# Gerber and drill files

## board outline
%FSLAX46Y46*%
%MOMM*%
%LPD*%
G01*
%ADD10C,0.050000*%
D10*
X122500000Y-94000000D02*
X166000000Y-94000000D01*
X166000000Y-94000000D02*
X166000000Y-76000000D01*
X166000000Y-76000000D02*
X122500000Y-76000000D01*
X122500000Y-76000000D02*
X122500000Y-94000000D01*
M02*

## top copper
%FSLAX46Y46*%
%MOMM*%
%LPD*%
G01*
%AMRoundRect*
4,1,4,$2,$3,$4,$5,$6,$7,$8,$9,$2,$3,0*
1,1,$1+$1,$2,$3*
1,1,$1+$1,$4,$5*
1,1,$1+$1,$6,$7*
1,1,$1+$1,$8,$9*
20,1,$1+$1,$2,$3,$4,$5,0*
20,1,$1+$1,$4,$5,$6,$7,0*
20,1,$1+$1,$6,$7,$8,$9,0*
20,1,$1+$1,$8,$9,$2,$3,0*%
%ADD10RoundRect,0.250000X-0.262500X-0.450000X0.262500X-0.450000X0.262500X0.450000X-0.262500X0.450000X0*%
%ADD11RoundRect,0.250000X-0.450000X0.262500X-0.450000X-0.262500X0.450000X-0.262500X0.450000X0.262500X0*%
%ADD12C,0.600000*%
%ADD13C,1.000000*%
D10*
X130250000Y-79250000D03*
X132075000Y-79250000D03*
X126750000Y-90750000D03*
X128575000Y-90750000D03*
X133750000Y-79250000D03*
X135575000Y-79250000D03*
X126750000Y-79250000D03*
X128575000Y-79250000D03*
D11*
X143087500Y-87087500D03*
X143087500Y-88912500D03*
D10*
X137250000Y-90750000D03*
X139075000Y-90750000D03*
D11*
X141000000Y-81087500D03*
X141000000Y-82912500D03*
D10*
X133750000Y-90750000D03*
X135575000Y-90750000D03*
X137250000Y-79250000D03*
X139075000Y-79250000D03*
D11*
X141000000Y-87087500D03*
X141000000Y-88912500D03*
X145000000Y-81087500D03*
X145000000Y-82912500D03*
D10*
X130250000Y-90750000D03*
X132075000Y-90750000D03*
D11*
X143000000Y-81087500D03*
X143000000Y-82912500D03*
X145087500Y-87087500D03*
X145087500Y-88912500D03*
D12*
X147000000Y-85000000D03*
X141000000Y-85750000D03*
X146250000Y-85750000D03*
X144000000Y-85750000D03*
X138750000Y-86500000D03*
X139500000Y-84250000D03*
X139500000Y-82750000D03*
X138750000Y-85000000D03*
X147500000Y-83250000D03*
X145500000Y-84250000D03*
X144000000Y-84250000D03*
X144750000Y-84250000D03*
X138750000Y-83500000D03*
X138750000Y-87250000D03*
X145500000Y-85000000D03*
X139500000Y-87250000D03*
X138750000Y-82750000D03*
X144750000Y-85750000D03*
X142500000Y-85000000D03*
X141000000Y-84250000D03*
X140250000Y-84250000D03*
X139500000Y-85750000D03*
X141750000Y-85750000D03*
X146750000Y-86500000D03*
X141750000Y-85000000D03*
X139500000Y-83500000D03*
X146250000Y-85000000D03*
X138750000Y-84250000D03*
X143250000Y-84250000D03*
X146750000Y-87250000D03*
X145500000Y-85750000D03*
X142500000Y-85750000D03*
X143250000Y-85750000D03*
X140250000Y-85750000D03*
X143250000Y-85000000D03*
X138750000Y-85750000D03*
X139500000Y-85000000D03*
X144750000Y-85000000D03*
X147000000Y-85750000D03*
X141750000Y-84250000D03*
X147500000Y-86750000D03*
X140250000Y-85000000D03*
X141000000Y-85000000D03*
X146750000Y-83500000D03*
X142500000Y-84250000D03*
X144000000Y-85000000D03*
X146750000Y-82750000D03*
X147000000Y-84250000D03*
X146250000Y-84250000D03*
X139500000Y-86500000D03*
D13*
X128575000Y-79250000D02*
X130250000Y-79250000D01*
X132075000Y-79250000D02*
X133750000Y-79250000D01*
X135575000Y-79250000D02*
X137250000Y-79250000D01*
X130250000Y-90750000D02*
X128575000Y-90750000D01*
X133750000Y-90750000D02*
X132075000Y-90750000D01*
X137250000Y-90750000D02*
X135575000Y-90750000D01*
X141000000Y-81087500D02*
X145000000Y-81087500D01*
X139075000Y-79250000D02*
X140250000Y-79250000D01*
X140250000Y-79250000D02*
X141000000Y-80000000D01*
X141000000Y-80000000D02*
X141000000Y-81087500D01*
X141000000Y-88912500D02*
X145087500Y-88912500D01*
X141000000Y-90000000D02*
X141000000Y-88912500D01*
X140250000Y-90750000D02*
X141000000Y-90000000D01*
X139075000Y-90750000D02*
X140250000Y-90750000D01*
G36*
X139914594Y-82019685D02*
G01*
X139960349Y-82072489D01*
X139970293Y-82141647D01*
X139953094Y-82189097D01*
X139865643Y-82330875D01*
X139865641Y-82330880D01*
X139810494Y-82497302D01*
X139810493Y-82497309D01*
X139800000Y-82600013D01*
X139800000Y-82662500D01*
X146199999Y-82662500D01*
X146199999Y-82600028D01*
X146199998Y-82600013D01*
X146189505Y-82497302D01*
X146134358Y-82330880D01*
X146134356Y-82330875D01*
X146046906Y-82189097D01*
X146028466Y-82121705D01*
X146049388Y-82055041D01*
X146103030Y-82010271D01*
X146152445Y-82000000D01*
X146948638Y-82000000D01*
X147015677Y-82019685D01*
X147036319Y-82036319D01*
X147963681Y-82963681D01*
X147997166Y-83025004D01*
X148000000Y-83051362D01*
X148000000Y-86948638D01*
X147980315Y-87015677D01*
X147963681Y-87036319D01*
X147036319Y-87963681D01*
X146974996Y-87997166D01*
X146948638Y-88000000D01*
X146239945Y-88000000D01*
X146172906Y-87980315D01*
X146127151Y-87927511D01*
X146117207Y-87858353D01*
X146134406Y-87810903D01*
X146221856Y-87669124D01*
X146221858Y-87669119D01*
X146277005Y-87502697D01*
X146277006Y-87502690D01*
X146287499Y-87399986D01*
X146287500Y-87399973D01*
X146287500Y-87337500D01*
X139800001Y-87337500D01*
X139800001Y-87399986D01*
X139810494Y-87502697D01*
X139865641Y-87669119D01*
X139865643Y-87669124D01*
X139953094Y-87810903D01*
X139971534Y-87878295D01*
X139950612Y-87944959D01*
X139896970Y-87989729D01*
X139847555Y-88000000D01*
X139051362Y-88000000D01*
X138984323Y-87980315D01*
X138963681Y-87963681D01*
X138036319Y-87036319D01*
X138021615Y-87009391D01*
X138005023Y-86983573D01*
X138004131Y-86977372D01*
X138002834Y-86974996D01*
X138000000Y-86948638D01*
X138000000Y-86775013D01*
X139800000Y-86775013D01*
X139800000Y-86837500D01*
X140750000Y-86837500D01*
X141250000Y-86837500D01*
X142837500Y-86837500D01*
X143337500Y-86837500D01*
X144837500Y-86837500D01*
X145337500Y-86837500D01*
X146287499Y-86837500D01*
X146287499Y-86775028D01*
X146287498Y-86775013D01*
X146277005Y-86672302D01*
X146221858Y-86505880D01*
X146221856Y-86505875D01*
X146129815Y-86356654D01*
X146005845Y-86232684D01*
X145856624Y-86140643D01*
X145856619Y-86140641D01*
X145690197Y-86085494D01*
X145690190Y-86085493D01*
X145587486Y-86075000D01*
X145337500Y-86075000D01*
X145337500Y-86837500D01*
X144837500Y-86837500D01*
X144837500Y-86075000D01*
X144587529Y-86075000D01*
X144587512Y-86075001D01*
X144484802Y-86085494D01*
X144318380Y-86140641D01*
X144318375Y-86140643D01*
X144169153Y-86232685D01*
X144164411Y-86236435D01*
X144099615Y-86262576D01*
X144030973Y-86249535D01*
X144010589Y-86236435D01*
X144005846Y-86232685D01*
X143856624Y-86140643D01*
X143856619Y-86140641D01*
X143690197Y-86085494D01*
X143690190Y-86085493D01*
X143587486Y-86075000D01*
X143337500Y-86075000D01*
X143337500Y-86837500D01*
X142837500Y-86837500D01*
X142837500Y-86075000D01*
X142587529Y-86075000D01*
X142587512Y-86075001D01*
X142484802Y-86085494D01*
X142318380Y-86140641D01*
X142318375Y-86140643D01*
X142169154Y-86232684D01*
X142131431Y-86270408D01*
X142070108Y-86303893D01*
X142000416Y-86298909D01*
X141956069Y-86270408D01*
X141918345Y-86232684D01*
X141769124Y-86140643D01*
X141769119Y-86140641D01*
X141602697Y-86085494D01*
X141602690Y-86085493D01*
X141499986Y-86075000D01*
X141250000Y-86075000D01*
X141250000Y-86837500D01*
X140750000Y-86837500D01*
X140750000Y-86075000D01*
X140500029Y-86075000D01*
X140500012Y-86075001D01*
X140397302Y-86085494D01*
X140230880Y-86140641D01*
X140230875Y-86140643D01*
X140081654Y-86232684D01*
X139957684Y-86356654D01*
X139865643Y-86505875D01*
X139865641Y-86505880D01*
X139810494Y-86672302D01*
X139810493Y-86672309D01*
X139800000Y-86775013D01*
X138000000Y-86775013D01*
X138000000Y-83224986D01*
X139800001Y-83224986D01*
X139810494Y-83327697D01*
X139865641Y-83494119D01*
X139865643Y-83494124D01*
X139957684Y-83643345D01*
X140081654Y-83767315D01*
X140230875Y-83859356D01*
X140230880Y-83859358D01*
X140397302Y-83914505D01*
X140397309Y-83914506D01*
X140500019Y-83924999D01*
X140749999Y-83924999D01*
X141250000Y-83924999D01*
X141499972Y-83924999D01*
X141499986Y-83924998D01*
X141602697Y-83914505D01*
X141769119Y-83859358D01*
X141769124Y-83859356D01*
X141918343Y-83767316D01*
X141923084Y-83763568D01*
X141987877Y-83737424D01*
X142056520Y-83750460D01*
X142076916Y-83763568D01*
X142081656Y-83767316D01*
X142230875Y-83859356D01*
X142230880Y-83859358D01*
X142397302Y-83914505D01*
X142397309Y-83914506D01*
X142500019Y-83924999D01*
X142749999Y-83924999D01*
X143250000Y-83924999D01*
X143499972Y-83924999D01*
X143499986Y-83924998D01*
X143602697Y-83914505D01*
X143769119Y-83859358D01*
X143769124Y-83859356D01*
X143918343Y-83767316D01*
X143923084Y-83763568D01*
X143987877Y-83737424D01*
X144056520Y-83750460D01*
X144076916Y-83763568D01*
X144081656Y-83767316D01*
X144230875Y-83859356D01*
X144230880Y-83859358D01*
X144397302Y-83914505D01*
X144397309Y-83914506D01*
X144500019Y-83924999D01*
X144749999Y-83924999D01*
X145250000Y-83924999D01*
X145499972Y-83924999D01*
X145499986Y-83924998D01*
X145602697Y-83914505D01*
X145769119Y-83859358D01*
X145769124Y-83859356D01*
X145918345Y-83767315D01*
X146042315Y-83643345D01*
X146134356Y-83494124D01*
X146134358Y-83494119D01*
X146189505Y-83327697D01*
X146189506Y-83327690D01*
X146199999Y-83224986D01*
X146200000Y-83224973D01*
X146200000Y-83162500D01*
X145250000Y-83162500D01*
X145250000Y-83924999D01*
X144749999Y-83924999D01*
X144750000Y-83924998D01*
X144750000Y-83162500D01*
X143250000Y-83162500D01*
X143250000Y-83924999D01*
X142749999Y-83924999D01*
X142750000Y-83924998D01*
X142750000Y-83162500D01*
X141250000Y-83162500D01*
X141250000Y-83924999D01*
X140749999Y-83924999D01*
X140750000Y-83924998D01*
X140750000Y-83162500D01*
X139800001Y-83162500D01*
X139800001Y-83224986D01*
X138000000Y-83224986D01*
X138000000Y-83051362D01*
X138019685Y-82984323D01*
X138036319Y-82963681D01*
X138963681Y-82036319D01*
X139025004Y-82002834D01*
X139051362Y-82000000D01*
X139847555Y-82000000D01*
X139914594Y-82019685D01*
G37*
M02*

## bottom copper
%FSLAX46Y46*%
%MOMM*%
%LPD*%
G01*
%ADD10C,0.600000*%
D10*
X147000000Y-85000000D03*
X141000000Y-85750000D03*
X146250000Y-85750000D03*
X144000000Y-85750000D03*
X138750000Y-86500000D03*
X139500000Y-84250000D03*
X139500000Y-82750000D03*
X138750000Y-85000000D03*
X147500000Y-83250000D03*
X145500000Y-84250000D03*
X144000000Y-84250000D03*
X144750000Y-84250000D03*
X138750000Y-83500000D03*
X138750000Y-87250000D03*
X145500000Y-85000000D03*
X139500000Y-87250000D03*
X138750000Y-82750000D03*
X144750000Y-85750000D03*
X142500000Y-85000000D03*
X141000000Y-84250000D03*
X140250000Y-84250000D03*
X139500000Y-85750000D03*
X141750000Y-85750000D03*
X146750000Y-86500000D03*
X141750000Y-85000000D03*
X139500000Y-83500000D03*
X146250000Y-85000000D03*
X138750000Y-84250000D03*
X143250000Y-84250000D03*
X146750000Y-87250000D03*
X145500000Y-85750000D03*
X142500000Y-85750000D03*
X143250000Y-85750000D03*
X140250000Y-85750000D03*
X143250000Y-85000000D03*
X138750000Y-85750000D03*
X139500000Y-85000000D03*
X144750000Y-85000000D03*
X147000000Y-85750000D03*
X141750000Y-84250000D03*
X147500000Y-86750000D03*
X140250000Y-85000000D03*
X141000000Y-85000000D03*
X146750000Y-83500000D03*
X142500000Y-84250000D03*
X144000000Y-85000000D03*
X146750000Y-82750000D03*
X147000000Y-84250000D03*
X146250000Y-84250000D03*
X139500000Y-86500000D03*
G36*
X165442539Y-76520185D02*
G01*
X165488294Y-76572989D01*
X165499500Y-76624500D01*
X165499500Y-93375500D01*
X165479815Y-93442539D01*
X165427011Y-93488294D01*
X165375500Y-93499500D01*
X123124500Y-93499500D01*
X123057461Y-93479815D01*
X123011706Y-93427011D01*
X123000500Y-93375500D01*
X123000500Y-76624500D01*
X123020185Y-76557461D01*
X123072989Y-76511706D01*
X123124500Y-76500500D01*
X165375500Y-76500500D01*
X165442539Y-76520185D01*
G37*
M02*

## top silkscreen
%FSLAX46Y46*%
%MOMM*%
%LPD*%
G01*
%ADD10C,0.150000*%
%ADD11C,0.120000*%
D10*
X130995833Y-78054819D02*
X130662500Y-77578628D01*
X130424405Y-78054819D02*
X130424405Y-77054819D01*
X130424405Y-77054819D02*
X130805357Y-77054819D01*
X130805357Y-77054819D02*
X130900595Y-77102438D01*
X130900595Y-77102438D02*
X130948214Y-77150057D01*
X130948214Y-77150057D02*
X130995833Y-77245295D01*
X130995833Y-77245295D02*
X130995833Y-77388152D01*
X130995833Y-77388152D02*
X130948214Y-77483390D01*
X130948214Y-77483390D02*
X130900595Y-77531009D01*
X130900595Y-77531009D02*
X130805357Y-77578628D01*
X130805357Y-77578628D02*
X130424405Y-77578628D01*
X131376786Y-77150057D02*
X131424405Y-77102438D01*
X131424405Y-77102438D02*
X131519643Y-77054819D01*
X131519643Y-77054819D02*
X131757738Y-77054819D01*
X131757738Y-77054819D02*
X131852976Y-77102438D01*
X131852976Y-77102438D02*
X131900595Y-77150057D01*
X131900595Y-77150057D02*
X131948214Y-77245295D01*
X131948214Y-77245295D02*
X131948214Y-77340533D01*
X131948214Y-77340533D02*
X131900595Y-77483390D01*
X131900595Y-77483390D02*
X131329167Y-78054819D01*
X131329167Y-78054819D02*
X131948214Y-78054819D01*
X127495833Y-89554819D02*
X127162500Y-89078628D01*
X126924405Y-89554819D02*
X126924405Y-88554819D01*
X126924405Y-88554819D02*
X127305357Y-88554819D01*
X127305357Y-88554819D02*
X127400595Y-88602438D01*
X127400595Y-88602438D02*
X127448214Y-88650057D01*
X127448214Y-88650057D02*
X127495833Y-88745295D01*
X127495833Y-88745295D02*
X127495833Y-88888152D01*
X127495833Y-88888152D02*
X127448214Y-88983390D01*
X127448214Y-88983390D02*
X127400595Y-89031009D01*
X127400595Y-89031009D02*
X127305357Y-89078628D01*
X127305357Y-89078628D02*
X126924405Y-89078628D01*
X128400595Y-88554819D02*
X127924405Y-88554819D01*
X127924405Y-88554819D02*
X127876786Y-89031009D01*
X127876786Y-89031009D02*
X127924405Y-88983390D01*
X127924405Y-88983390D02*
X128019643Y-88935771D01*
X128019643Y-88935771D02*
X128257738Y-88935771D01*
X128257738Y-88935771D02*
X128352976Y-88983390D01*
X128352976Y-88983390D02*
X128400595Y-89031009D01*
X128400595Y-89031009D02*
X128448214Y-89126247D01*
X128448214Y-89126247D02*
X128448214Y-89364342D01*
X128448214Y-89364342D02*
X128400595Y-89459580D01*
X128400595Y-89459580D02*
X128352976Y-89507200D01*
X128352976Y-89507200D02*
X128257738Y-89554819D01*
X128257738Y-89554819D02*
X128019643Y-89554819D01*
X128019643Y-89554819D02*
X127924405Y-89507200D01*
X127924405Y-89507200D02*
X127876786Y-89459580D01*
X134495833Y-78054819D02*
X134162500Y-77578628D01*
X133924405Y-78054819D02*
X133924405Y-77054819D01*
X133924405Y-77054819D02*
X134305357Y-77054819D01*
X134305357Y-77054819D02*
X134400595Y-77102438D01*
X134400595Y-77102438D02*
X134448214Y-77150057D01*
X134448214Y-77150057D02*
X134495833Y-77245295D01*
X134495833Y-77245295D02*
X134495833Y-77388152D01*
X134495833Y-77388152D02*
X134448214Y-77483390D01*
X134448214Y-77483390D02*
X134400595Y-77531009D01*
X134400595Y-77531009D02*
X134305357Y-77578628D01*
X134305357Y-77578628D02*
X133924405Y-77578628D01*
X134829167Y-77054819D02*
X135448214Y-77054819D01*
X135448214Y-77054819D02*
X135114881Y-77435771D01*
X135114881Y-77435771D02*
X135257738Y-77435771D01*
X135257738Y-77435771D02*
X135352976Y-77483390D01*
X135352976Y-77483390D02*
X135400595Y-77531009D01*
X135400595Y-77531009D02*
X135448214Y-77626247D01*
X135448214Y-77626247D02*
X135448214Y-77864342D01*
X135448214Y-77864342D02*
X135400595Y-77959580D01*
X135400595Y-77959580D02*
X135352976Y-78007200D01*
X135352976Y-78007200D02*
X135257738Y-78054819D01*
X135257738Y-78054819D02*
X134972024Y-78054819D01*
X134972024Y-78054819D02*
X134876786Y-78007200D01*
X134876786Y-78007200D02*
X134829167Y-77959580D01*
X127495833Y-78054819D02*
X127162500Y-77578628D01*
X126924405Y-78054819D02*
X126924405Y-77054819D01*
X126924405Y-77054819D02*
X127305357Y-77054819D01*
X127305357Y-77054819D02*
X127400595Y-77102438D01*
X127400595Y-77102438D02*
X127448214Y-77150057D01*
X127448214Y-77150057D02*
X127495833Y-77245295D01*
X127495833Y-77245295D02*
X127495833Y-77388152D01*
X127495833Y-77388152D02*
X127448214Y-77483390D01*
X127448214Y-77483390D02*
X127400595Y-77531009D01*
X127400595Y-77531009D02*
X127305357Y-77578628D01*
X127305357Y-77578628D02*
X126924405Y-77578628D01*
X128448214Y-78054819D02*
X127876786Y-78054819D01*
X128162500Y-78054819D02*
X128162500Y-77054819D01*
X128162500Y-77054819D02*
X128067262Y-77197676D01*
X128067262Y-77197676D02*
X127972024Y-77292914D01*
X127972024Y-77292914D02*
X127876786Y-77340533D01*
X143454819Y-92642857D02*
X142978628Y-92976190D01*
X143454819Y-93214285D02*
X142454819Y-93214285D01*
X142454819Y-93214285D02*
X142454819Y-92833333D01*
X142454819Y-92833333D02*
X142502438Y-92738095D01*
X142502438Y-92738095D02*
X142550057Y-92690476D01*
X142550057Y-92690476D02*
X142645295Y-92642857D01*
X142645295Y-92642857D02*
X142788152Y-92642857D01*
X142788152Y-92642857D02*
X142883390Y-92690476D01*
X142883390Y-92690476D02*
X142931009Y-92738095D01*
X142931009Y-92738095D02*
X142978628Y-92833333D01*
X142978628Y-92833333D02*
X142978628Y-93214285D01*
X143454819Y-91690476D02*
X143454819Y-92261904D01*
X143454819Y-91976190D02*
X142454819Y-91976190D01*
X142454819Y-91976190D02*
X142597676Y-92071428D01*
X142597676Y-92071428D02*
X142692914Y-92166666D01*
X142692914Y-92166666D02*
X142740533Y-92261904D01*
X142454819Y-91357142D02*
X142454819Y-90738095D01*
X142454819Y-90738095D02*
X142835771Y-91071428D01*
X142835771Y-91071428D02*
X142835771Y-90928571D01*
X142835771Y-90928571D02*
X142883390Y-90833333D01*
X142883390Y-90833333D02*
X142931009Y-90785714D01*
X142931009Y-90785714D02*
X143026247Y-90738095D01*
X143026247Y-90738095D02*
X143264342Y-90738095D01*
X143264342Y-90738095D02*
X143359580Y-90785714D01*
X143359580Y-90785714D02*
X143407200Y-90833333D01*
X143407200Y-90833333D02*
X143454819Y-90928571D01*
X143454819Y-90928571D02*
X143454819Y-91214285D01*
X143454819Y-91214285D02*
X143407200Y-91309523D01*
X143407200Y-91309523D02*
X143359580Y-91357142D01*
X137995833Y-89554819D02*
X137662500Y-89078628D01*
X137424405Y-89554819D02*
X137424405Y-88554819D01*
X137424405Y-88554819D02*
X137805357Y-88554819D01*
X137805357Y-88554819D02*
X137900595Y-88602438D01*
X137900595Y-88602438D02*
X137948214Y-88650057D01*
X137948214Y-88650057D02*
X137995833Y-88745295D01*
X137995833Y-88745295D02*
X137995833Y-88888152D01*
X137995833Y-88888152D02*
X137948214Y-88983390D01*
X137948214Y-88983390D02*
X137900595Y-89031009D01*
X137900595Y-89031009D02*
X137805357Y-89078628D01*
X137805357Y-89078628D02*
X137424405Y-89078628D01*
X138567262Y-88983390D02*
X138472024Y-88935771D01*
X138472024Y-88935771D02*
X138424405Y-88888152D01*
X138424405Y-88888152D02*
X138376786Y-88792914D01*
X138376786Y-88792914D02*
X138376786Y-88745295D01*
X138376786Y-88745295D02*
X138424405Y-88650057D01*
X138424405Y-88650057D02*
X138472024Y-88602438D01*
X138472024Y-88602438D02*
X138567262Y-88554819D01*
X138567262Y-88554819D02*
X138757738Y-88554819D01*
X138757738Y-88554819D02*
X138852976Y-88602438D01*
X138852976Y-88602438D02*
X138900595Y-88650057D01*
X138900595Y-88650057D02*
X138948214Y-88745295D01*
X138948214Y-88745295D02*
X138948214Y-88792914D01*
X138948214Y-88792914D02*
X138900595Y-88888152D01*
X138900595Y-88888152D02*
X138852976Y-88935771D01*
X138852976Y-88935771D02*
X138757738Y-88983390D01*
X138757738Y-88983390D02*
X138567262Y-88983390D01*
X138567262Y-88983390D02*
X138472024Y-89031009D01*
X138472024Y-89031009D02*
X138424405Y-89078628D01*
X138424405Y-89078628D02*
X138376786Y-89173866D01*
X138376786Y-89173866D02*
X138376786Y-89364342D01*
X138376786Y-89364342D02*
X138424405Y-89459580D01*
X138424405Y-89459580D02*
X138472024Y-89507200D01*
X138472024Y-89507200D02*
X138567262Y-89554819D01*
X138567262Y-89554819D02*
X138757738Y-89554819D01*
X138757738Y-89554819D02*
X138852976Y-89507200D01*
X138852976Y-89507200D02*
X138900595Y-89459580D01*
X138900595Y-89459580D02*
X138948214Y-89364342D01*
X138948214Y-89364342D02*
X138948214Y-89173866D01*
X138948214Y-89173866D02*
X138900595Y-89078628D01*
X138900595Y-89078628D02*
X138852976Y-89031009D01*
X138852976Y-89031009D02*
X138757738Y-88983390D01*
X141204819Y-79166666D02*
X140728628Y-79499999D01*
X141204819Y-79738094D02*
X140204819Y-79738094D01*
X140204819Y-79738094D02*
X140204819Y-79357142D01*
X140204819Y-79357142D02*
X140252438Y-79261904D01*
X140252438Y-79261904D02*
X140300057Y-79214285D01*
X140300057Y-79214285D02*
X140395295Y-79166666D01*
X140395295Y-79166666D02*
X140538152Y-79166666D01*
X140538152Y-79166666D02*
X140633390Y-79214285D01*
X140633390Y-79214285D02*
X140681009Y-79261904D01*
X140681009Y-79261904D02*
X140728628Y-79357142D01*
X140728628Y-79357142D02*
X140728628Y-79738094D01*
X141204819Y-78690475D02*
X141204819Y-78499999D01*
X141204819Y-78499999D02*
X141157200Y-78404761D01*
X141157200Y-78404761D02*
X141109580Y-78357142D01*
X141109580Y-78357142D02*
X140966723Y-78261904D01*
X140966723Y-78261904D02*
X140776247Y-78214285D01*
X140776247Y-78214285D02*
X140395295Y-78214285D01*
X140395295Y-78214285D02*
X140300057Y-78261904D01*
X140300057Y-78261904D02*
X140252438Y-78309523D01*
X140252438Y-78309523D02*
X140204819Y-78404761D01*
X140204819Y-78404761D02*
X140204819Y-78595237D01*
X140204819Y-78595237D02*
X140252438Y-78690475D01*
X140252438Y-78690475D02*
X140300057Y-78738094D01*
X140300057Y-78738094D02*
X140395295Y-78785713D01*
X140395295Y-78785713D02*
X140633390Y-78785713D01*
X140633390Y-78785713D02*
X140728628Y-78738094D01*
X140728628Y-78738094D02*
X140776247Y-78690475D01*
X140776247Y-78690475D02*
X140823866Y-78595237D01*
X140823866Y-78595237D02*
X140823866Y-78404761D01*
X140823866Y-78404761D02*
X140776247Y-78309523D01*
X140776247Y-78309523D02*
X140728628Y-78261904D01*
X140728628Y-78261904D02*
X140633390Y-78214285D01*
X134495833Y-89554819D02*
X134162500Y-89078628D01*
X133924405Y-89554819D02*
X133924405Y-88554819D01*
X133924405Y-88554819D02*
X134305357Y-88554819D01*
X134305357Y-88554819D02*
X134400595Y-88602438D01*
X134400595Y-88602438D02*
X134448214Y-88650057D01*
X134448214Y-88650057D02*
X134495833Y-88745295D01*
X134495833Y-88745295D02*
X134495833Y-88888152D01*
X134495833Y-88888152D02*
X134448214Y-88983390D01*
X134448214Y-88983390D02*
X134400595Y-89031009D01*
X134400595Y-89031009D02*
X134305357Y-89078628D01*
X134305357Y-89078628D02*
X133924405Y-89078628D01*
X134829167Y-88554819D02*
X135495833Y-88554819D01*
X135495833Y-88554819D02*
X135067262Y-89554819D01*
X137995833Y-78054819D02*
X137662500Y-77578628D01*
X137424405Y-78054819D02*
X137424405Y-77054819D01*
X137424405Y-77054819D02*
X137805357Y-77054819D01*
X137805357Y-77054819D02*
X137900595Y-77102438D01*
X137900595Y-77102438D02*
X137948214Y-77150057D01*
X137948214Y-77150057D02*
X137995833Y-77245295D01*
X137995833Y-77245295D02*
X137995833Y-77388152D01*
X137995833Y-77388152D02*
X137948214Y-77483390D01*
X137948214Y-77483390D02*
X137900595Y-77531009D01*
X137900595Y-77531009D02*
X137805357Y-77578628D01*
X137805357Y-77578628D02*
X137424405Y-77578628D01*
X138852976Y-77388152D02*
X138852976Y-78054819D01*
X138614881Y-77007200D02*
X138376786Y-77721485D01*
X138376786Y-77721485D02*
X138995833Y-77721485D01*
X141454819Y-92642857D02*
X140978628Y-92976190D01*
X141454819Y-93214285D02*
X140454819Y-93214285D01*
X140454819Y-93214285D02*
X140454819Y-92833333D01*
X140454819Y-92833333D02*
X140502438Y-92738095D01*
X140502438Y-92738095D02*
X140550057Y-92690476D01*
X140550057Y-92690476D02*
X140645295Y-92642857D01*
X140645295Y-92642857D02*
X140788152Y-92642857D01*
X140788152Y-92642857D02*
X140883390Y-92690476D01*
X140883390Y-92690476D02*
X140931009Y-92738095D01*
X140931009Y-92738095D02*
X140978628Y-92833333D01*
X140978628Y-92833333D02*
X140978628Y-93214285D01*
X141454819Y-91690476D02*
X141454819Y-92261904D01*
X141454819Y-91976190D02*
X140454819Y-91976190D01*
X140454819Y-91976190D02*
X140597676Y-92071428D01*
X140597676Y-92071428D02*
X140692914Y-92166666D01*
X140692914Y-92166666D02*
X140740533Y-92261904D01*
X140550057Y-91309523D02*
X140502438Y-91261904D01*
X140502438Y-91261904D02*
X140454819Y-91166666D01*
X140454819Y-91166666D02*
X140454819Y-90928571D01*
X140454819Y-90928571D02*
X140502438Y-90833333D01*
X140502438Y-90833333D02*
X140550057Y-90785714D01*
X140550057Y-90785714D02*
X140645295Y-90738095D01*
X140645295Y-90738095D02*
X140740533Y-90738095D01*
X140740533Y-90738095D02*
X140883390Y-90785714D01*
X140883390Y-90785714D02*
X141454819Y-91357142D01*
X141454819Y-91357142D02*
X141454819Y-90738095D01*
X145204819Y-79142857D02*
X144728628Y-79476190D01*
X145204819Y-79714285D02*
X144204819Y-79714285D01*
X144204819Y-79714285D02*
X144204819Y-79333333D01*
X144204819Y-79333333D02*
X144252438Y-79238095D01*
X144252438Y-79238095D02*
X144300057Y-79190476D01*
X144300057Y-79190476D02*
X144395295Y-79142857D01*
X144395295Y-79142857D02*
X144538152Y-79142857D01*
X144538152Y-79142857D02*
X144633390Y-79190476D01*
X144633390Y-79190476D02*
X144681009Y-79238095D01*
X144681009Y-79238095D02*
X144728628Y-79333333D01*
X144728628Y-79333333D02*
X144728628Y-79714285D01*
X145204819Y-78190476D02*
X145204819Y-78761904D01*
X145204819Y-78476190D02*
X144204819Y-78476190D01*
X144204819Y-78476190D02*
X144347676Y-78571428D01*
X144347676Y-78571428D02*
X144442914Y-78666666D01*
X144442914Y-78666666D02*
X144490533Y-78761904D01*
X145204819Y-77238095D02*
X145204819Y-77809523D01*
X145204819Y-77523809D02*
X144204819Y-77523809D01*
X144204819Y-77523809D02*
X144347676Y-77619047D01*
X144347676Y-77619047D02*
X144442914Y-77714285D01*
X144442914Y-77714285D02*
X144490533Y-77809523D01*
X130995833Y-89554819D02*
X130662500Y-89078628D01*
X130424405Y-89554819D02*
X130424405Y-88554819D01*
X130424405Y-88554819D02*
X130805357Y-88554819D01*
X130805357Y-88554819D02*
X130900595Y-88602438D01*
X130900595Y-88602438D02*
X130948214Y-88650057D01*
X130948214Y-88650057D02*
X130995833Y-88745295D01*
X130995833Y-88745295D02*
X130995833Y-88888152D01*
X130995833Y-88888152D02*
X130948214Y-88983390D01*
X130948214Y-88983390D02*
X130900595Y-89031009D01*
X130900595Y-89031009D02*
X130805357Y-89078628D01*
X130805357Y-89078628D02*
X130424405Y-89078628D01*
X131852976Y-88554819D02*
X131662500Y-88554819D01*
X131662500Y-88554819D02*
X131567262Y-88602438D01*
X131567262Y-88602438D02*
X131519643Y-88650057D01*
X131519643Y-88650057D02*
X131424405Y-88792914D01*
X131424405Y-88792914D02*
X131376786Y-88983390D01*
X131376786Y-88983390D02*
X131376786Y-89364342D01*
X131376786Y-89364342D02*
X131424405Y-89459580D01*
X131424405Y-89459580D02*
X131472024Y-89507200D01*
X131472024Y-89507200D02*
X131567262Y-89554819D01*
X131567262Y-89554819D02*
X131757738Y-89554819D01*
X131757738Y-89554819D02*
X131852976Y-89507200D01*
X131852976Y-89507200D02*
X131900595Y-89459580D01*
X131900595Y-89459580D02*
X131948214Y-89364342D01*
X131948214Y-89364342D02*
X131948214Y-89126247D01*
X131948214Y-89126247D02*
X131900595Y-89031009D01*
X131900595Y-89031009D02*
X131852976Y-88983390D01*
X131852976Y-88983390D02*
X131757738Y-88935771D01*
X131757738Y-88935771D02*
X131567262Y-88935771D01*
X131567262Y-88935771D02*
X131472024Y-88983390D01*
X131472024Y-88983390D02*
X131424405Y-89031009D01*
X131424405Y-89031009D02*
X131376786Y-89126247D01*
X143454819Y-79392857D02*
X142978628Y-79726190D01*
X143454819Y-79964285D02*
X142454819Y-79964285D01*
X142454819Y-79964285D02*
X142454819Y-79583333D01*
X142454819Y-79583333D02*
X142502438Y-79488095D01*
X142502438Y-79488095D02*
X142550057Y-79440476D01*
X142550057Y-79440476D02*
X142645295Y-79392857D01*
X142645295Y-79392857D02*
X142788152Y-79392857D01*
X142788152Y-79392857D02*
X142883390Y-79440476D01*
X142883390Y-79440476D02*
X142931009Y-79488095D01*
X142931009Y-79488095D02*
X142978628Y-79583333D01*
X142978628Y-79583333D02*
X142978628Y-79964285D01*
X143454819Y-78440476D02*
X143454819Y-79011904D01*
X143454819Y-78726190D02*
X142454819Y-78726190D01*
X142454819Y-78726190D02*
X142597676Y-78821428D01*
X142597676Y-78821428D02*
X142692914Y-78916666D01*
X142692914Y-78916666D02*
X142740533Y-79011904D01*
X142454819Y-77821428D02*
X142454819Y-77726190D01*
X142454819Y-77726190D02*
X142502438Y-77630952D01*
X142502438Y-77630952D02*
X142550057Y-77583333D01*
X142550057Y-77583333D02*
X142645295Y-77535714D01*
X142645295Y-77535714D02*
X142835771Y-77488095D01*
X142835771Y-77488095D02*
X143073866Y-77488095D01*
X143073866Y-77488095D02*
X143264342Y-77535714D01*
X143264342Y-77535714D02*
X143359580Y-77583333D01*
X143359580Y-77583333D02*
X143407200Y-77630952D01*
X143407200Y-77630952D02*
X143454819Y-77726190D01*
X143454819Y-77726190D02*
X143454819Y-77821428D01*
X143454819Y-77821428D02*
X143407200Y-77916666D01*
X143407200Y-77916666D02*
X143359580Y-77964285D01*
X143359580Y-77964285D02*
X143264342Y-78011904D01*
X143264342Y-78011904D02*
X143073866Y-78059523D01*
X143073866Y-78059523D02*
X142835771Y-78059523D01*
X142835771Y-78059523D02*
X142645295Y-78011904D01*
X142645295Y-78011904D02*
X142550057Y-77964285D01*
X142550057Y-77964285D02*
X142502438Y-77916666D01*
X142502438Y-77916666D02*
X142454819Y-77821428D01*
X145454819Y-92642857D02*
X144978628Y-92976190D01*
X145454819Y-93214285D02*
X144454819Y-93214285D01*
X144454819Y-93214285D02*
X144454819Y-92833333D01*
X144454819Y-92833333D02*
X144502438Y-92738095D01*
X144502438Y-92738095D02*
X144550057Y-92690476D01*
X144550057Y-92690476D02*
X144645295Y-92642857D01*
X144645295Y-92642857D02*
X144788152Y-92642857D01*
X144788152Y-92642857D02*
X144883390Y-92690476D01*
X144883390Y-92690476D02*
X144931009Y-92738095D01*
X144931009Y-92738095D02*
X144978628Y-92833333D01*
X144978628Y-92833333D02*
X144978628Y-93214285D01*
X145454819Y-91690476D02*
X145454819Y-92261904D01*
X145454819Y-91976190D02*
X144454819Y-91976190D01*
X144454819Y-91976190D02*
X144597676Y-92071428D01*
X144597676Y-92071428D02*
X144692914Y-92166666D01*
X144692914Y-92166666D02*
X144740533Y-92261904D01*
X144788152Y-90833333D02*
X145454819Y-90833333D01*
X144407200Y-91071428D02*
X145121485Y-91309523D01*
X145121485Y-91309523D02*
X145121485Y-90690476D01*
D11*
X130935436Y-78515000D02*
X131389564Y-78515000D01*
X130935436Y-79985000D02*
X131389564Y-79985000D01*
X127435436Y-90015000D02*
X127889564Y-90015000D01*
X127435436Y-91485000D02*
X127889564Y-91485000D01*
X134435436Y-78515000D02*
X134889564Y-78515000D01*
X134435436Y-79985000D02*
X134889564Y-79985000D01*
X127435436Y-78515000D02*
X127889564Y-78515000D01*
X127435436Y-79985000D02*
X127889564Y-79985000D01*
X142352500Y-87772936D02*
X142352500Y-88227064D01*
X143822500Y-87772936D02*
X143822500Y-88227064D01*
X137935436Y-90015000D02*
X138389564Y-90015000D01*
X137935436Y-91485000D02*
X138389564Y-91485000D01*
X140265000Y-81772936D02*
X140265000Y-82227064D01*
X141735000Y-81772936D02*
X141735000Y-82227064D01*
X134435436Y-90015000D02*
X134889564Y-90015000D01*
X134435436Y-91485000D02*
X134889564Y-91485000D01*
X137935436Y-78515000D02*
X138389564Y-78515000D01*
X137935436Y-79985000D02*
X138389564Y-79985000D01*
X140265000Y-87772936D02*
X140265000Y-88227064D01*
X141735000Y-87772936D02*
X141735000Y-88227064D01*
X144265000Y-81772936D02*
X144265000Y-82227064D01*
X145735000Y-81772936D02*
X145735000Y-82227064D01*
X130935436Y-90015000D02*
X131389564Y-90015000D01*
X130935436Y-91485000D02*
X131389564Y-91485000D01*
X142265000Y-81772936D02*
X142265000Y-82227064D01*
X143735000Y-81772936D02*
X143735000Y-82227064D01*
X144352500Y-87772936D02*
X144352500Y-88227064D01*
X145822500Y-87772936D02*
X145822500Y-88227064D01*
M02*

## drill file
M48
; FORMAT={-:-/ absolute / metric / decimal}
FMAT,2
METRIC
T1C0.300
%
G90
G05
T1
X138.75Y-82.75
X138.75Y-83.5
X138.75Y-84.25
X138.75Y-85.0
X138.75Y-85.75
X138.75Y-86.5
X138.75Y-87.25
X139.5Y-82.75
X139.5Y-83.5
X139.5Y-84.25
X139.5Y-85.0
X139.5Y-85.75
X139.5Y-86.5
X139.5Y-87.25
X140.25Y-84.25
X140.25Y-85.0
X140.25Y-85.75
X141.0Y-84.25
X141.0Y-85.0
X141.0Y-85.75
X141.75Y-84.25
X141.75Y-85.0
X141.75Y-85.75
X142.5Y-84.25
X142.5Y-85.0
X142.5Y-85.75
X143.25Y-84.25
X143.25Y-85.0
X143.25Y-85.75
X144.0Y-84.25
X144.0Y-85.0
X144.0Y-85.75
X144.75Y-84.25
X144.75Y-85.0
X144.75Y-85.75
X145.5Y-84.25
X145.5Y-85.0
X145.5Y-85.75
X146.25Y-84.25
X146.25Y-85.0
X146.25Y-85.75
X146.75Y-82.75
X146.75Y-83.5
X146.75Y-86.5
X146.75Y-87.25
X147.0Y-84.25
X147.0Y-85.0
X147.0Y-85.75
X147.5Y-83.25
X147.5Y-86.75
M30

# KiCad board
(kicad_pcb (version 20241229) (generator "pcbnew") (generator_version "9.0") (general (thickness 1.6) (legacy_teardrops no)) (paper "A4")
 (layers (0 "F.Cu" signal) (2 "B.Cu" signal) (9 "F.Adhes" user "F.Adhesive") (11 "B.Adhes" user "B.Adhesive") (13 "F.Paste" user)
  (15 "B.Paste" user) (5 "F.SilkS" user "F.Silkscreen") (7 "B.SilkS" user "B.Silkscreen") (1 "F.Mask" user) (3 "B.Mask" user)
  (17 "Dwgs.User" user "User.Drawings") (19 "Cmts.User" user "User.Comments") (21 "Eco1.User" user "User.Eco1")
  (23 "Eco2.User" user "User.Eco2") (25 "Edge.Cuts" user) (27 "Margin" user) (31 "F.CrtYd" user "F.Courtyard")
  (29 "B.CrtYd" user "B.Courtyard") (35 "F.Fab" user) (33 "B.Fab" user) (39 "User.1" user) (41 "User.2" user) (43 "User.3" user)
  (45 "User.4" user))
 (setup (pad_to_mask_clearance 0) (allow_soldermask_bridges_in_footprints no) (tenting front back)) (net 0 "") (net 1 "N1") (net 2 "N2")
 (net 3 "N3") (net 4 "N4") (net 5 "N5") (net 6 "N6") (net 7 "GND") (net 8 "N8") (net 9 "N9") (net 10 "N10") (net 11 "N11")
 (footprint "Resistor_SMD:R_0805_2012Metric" (layer "F.Cu") (at 131.1625 79.25)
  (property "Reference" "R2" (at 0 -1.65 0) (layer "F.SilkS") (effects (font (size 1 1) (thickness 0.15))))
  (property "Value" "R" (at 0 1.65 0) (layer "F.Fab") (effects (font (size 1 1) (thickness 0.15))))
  (fp_line (start -0.227064 -0.735) (end 0.227064 -0.735) (stroke (width 0.12) (type solid)) (layer "F.SilkS"))
  (fp_line (start -0.227064 0.735) (end 0.227064 0.735) (stroke (width 0.12) (type solid)) (layer "F.SilkS"))
  (pad "1" smd roundrect (at -0.9125 0) (size 1.025 1.4) (layers "F.Cu" "F.Mask" "F.Paste") (roundrect_rratio 0.243902) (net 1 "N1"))
  (pad "2" smd roundrect (at 0.9125 0) (size 1.025 1.4) (layers "F.Cu" "F.Mask" "F.Paste") (roundrect_rratio 0.243902) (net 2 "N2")))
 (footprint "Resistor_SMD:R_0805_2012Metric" (layer "F.Cu") (at 127.6625 90.75)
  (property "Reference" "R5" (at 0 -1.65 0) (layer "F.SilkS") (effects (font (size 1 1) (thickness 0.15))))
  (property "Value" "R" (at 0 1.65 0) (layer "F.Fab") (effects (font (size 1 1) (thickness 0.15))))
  (fp_line (start -0.227064 -0.735) (end 0.227064 -0.735) (stroke (width 0.12) (type solid)) (layer "F.SilkS"))
  (fp_line (start -0.227064 0.735) (end 0.227064 0.735) (stroke (width 0.12) (type solid)) (layer "F.SilkS"))
  (pad "1" smd roundrect (at -0.9125 0) (size 1.025 1.4) (layers "F.Cu" "F.Mask" "F.Paste") (roundrect_rratio 0.243902) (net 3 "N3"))
  (pad "2" smd roundrect (at 0.9125 0) (size 1.025 1.4) (layers "F.Cu" "F.Mask" "F.Paste") (roundrect_rratio 0.243902) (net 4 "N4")))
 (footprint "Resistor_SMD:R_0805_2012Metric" (layer "F.Cu") (at 134.6625 79.25)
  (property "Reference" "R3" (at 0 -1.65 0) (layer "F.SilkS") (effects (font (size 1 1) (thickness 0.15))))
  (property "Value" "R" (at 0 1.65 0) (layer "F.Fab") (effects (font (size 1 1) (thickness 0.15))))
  (fp_line (start -0.227064 -0.735) (end 0.227064 -0.735) (stroke (width 0.12) (type solid)) (layer "F.SilkS"))
  (fp_line (start -0.227064 0.735) (end 0.227064 0.735) (stroke (width 0.12) (type solid)) (layer "F.SilkS"))
  (pad "1" smd roundrect (at -0.9125 0) (size 1.025 1.4) (layers "F.Cu" "F.Mask" "F.Paste") (roundrect_rratio 0.243902) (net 2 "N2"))
  (pad "2" smd roundrect (at 0.9125 0) (size 1.025 1.4) (layers "F.Cu" "F.Mask" "F.Paste") (roundrect_rratio 0.243902) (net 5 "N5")))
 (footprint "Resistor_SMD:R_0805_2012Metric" (layer "F.Cu") (at 127.6625 79.25)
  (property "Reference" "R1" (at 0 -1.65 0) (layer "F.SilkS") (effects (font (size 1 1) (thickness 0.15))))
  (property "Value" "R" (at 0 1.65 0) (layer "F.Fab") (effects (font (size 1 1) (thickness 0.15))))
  (fp_line (start -0.227064 -0.735) (end 0.227064 -0.735) (stroke (width 0.12) (type solid)) (layer "F.SilkS"))
  (fp_line (start -0.227064 0.735) (end 0.227064 0.735) (stroke (width 0.12) (type solid)) (layer "F.SilkS"))
  (pad "1" smd roundrect (at -0.9125 0) (size 1.025 1.4) (layers "F.Cu" "F.Mask" "F.Paste") (roundrect_rratio 0.243902) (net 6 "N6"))
  (pad "2" smd roundrect (at 0.9125 0) (size 1.025 1.4) (layers "F.Cu" "F.Mask" "F.Paste") (roundrect_rratio 0.243902) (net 1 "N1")))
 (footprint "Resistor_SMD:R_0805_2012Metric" (layer "F.Cu") (at 143.0875 88 -90)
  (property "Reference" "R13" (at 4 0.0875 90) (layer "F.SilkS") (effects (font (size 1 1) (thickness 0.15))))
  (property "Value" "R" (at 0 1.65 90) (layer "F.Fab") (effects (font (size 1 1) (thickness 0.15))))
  (fp_line (start -0.227064 0.735) (end 0.227064 0.735) (stroke (width 0.12) (type solid)) (layer "F.SilkS"))
  (fp_line (start -0.227064 -0.735) (end 0.227064 -0.735) (stroke (width 0.12) (type solid)) (layer "F.SilkS"))
  (pad "1" smd roundrect (at -0.9125 0 270) (size 1.025 1.4) (layers "F.Cu" "F.Mask" "F.Paste") (roundrect_rratio 0.243902) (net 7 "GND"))
  (pad "2" smd roundrect (at 0.9125 0 270) (size 1.025 1.4) (layers "F.Cu" "F.Mask" "F.Paste") (roundrect_rratio 0.243902) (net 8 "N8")))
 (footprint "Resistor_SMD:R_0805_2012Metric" (layer "F.Cu") (at 138.1625 90.75)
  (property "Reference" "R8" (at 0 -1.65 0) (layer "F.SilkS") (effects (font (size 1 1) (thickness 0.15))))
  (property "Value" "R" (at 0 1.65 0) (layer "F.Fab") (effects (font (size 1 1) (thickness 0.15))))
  (fp_line (start -0.227064 -0.735) (end 0.227064 -0.735) (stroke (width 0.12) (type solid)) (layer "F.SilkS"))
  (fp_line (start -0.227064 0.735) (end 0.227064 0.735) (stroke (width 0.12) (type solid)) (layer "F.SilkS"))
  (pad "1" smd roundrect (at -0.9125 0) (size 1.025 1.4) (layers "F.Cu" "F.Mask" "F.Paste") (roundrect_rratio 0.243902) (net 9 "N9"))
  (pad "2" smd roundrect (at 0.9125 0) (size 1.025 1.4) (layers "F.Cu" "F.Mask" "F.Paste") (roundrect_rratio 0.243902) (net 8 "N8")))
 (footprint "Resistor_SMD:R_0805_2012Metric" (layer "F.Cu") (at 141 82 -90)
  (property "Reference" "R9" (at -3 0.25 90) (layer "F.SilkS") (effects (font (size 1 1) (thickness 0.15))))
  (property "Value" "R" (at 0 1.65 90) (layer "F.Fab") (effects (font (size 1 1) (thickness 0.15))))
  (fp_line (start -0.227064 0.735) (end 0.227064 0.735) (stroke (width 0.12) (type solid)) (layer "F.SilkS"))
  (fp_line (start -0.227064 -0.735) (end 0.227064 -0.735) (stroke (width 0.12) (type solid)) (layer "F.SilkS"))
  (pad "1" smd roundrect (at -0.9125 0 270) (size 1.025 1.4) (layers "F.Cu" "F.Mask" "F.Paste") (roundrect_rratio 0.243902) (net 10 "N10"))
  (pad "2" smd roundrect (at 0.9125 0 270) (size 1.025 1.4) (layers "F.Cu" "F.Mask" "F.Paste") (roundrect_rratio 0.243902) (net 7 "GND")))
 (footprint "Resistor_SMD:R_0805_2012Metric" (layer "F.Cu") (at 134.6625 90.75)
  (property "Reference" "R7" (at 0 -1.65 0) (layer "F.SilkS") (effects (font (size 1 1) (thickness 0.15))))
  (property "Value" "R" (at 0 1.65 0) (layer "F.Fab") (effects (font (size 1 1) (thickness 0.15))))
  (fp_line (start -0.227064 -0.735) (end 0.227064 -0.735) (stroke (width 0.12) (type solid)) (layer "F.SilkS"))
  (fp_line (start -0.227064 0.735) (end 0.227064 0.735) (stroke (width 0.12) (type solid)) (layer "F.SilkS"))
  (pad "1" smd roundrect (at -0.9125 0) (size 1.025 1.4) (layers "F.Cu" "F.Mask" "F.Paste") (roundrect_rratio 0.243902) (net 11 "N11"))
  (pad "2" smd roundrect (at 0.9125 0) (size 1.025 1.4) (layers "F.Cu" "F.Mask" "F.Paste") (roundrect_rratio 0.243902) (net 9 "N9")))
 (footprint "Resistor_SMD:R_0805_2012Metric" (layer "F.Cu") (at 138.1625 79.25)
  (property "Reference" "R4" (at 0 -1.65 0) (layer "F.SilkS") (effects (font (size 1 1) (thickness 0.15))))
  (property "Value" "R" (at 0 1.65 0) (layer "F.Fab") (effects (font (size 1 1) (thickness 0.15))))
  (fp_line (start -0.227064 -0.735) (end 0.227064 -0.735) (stroke (width 0.12) (type solid)) (layer "F.SilkS"))
  (fp_line (start -0.227064 0.735) (end 0.227064 0.735) (stroke (width 0.12) (type solid)) (layer "F.SilkS"))
  (pad "1" smd roundrect (at -0.9125 0) (size 1.025 1.4) (layers "F.Cu" "F.Mask" "F.Paste") (roundrect_rratio 0.243902) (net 5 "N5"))
  (pad "2" smd roundrect (at 0.9125 0) (size 1.025 1.4) (layers "F.Cu" "F.Mask" "F.Paste") (roundrect_rratio 0.243902) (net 10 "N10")))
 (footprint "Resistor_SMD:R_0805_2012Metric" (layer "F.Cu") (at 141 88 -90)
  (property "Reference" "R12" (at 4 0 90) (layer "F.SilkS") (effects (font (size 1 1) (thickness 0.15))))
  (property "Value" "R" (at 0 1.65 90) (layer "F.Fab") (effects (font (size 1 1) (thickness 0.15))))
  (fp_line (start -0.227064 0.735) (end 0.227064 0.735) (stroke (width 0.12) (type solid)) (layer "F.SilkS"))
  (fp_line (start -0.227064 -0.735) (end 0.227064 -0.735) (stroke (width 0.12) (type solid)) (layer "F.SilkS"))
  (pad "1" smd roundrect (at -0.9125 0 270) (size 1.025 1.4) (layers "F.Cu" "F.Mask" "F.Paste") (roundrect_rratio 0.243902) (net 7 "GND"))
  (pad "2" smd roundrect (at 0.9125 0 270) (size 1.025 1.4) (layers "F.Cu" "F.Mask" "F.Paste") (roundrect_rratio 0.243902) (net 8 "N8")))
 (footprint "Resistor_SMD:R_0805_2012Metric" (layer "F.Cu") (at 145 82 -90)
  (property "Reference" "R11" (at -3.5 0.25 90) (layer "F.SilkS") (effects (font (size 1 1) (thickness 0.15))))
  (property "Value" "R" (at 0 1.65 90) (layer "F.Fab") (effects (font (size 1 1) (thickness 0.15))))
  (fp_line (start -0.227064 0.735) (end 0.227064 0.735) (stroke (width 0.12) (type solid)) (layer "F.SilkS"))
  (fp_line (start -0.227064 -0.735) (end 0.227064 -0.735) (stroke (width 0.12) (type solid)) (layer "F.SilkS"))
  (pad "1" smd roundrect (at -0.9125 0 270) (size 1.025 1.4) (layers "F.Cu" "F.Mask" "F.Paste") (roundrect_rratio 0.243902) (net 10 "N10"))
  (pad "2" smd roundrect (at 0.9125 0 270) (size 1.025 1.4) (layers "F.Cu" "F.Mask" "F.Paste") (roundrect_rratio 0.243902) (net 7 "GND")))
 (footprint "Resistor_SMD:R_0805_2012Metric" (layer "F.Cu") (at 131.1625 90.75)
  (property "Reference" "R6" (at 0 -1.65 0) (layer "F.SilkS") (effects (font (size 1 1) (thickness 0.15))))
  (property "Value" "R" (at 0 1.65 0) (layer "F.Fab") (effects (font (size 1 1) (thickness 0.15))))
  (fp_line (start -0.227064 -0.735) (end 0.227064 -0.735) (stroke (width 0.12) (type solid)) (layer "F.SilkS"))
  (fp_line (start -0.227064 0.735) (end 0.227064 0.735) (stroke (width 0.12) (type solid)) (layer "F.SilkS"))
  (pad "1" smd roundrect (at -0.9125 0) (size 1.025 1.4) (layers "F.Cu" "F.Mask" "F.Paste") (roundrect_rratio 0.243902) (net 4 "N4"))
  (pad "2" smd roundrect (at 0.9125 0) (size 1.025 1.4) (layers "F.Cu" "F.Mask" "F.Paste") (roundrect_rratio 0.243902) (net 11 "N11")))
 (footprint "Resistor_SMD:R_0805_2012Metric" (layer "F.Cu") (at 143 82 -90)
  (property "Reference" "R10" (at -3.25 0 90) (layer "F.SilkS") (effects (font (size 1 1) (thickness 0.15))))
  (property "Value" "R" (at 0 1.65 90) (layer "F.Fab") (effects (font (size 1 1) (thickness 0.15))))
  (fp_line (start -0.227064 0.735) (end 0.227064 0.735) (stroke (width 0.12) (type solid)) (layer "F.SilkS"))
  (fp_line (start -0.227064 -0.735) (end 0.227064 -0.735) (stroke (width 0.12) (type solid)) (layer "F.SilkS"))
  (pad "1" smd roundrect (at -0.9125 0 270) (size 1.025 1.4) (layers "F.Cu" "F.Mask" "F.Paste") (roundrect_rratio 0.243902) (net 10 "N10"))
  (pad "2" smd roundrect (at 0.9125 0 270) (size 1.025 1.4) (layers "F.Cu" "F.Mask" "F.Paste") (roundrect_rratio 0.243902) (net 7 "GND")))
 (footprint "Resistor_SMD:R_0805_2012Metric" (layer "F.Cu") (at 145.0875 88 -90)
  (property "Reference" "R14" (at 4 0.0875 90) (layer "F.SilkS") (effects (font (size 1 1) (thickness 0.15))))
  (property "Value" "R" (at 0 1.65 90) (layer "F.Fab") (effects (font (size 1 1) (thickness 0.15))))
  (fp_line (start -0.227064 0.735) (end 0.227064 0.735) (stroke (width 0.12) (type solid)) (layer "F.SilkS"))
  (fp_line (start -0.227064 -0.735) (end 0.227064 -0.735) (stroke (width 0.12) (type solid)) (layer "F.SilkS"))
  (pad "1" smd roundrect (at -0.9125 0 270) (size 1.025 1.4) (layers "F.Cu" "F.Mask" "F.Paste") (roundrect_rratio 0.243902) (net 7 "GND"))
  (pad "2" smd roundrect (at 0.9125 0 270) (size 1.025 1.4) (layers "F.Cu" "F.Mask" "F.Paste") (roundrect_rratio 0.243902) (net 8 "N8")))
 (gr_line (start 122.5 94) (end 166 94) (stroke (width 0.05) (type default)) (layer "Edge.Cuts"))
 (gr_line (start 166 94) (end 166 76) (stroke (width 0.05) (type default)) (layer "Edge.Cuts"))
 (gr_line (start 166 76) (end 122.5 76) (stroke (width 0.05) (type default)) (layer "Edge.Cuts"))
 (gr_line (start 122.5 76) (end 122.5 94) (stroke (width 0.05) (type default)) (layer "Edge.Cuts"))
 (segment (start 128.575 79.25) (end 130.25 79.25) (width 1) (layer "F.Cu") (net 1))
 (segment (start 132.075 79.25) (end 133.75 79.25) (width 1) (layer "F.Cu") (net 2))
 (segment (start 135.575 79.25) (end 137.25 79.25) (width 1) (layer "F.Cu") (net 5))
 (segment (start 130.25 90.75) (end 128.575 90.75) (width 1) (layer "F.Cu") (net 4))
 (segment (start 133.75 90.75) (end 132.075 90.75) (width 1) (layer "F.Cu") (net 11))
 (segment (start 137.25 90.75) (end 135.575 90.75) (width 1) (layer "F.Cu") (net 9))
 (segment (start 141 81.0875) (end 145 81.0875) (width 1) (layer "F.Cu") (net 10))
 (segment (start 139.075 79.25) (end 140.25 79.25) (width 1) (layer "F.Cu") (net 10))
 (segment (start 140.25 79.25) (end 141 80) (width 1) (layer "F.Cu") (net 10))
 (segment (start 141 80) (end 141 81.0875) (width 1) (layer "F.Cu") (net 10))
 (via (at 147 85) (size 0.6) (drill 0.3) (layers "F.Cu" "B.Cu") (free yes) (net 7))
 (via (at 141 85.75) (size 0.6) (drill 0.3) (layers "F.Cu" "B.Cu") (free yes) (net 7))
 (via (at 146.25 85.75) (size 0.6) (drill 0.3) (layers "F.Cu" "B.Cu") (free yes) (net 7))
 (via (at 144 85.75) (size 0.6) (drill 0.3) (layers "F.Cu" "B.Cu") (free yes) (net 7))
 (via (at 138.75 86.5) (size 0.6) (drill 0.3) (layers "F.Cu" "B.Cu") (free yes) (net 7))
 (via (at 139.5 84.25) (size 0.6) (drill 0.3) (layers "F.Cu" "B.Cu") (free yes) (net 7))
 (via (at 139.5 82.75) (size 0.6) (drill 0.3) (layers "F.Cu" "B.Cu") (free yes) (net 7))
 (via (at 138.75 85) (size 0.6) (drill 0.3) (layers "F.Cu" "B.Cu") (free yes) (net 7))
 (via (at 147.5 83.25) (size 0.6) (drill 0.3) (layers "F.Cu" "B.Cu") (free yes) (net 7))
 (via (at 145.5 84.25) (size 0.6) (drill 0.3) (layers "F.Cu" "B.Cu") (free yes) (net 7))
 (via (at 144 84.25) (size 0.6) (drill 0.3) (layers "F.Cu" "B.Cu") (free yes) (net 7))
 (via (at 144.75 84.25) (size 0.6) (drill 0.3) (layers "F.Cu" "B.Cu") (free yes) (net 7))
 (via (at 138.75 83.5) (size 0.6) (drill 0.3) (layers "F.Cu" "B.Cu") (free yes) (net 7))
 (via (at 138.75 87.25) (size 0.6) (drill 0.3) (layers "F.Cu" "B.Cu") (free yes) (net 7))
 (via (at 145.5 85) (size 0.6) (drill 0.3) (layers "F.Cu" "B.Cu") (free yes) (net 7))
 (via (at 139.5 87.25) (size 0.6) (drill 0.3) (layers "F.Cu" "B.Cu") (free yes) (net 7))
 (via (at 138.75 82.75) (size 0.6) (drill 0.3) (layers "F.Cu" "B.Cu") (free yes) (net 7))
 (via (at 144.75 85.75) (size 0.6) (drill 0.3) (layers "F.Cu" "B.Cu") (free yes) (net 7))
 (via (at 142.5 85) (size 0.6) (drill 0.3) (layers "F.Cu" "B.Cu") (free yes) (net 7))
 (via (at 141 84.25) (size 0.6) (drill 0.3) (layers "F.Cu" "B.Cu") (free yes) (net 7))
 (via (at 140.25 84.25) (size 0.6) (drill 0.3) (layers "F.Cu" "B.Cu") (free yes) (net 7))
 (via (at 139.5 85.75) (size 0.6) (drill 0.3) (layers "F.Cu" "B.Cu") (free yes) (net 7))
 (via (at 141.75 85.75) (size 0.6) (drill 0.3) (layers "F.Cu" "B.Cu") (free yes) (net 7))
 (via (at 146.75 86.5) (size 0.6) (drill 0.3) (layers "F.Cu" "B.Cu") (free yes) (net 7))
 (via (at 141.75 85) (size 0.6) (drill 0.3) (layers "F.Cu" "B.Cu") (free yes) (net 7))
 (via (at 139.5 83.5) (size 0.6) (drill 0.3) (layers "F.Cu" "B.Cu") (free yes) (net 7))
 (via (at 146.25 85) (size 0.6) (drill 0.3) (layers "F.Cu" "B.Cu") (free yes) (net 7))
 (via (at 138.75 84.25) (size 0.6) (drill 0.3) (layers "F.Cu" "B.Cu") (free yes) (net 7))
 (via (at 143.25 84.25) (size 0.6) (drill 0.3) (layers "F.Cu" "B.Cu") (free yes) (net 7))
 (via (at 146.75 87.25) (size 0.6) (drill 0.3) (layers "F.Cu" "B.Cu") (free yes) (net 7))
 (via (at 145.5 85.75) (size 0.6) (drill 0.3) (layers "F.Cu" "B.Cu") (free yes) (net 7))
 (via (at 142.5 85.75) (size 0.6) (drill 0.3) (layers "F.Cu" "B.Cu") (free yes) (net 7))
 (via (at 143.25 85.75) (size 0.6) (drill 0.3) (layers "F.Cu" "B.Cu") (free yes) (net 7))
 (via (at 140.25 85.75) (size 0.6) (drill 0.3) (layers "F.Cu" "B.Cu") (free yes) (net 7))
 (via (at 143.25 85) (size 0.6) (drill 0.3) (layers "F.Cu" "B.Cu") (free yes) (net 7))
 (via (at 138.75 85.75) (size 0.6) (drill 0.3) (layers "F.Cu" "B.Cu") (free yes) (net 7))
 (via (at 139.5 85) (size 0.6) (drill 0.3) (layers "F.Cu" "B.Cu") (free yes) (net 7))
 (via (at 144.75 85) (size 0.6) (drill 0.3) (layers "F.Cu" "B.Cu") (free yes) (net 7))
 (via (at 147 85.75) (size 0.6) (drill 0.3) (layers "F.Cu" "B.Cu") (free yes) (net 7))
 (via (at 141.75 84.25) (size 0.6) (drill 0.3) (layers "F.Cu" "B.Cu") (free yes) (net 7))
 (via (at 147.5 86.75) (size 0.6) (drill 0.3) (layers "F.Cu" "B.Cu") (free yes) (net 7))
 (via (at 140.25 85) (size 0.6) (drill 0.3) (layers "F.Cu" "B.Cu") (free yes) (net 7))
 (via (at 141 85) (size 0.6) (drill 0.3) (layers "F.Cu" "B.Cu") (free yes) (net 7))
 (via (at 146.75 83.5) (size 0.6) (drill 0.3) (layers "F.Cu" "B.Cu") (free yes) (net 7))
 (via (at 142.5 84.25) (size 0.6) (drill 0.3) (layers "F.Cu" "B.Cu") (free yes) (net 7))
 (via (at 144 85) (size 0.6) (drill 0.3) (layers "F.Cu" "B.Cu") (free yes) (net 7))
 (via (at 146.75 82.75) (size 0.6) (drill 0.3) (layers "F.Cu" "B.Cu") (free yes) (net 7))
 (via (at 147 84.25) (size 0.6) (drill 0.3) (layers "F.Cu" "B.Cu") (free yes) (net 7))
 (via (at 146.25 84.25) (size 0.6) (drill 0.3) (layers "F.Cu" "B.Cu") (free yes) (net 7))
 (via (at 139.5 86.5) (size 0.6) (drill 0.3) (layers "F.Cu" "B.Cu") (free yes) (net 7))
 (segment (start 141 88.9125) (end 145.0875 88.9125) (width 1) (layer "F.Cu") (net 8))
 (segment (start 141 90) (end 141 88.9125) (width 1) (layer "F.Cu") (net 8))
 (segment (start 140.25 90.75) (end 141 90) (width 1) (layer "F.Cu") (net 8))
 (segment (start 139.075 90.75) (end 140.25 90.75) (width 1) (layer "F.Cu") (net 8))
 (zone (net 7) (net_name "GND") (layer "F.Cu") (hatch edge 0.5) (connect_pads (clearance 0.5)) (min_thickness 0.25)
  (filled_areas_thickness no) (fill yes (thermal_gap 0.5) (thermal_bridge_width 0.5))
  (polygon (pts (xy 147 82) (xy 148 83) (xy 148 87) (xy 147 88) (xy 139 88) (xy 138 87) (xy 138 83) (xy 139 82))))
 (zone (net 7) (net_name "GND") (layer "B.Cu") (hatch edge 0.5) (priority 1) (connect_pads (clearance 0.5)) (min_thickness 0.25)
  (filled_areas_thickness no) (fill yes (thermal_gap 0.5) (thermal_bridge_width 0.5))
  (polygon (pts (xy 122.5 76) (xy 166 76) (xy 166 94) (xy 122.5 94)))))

